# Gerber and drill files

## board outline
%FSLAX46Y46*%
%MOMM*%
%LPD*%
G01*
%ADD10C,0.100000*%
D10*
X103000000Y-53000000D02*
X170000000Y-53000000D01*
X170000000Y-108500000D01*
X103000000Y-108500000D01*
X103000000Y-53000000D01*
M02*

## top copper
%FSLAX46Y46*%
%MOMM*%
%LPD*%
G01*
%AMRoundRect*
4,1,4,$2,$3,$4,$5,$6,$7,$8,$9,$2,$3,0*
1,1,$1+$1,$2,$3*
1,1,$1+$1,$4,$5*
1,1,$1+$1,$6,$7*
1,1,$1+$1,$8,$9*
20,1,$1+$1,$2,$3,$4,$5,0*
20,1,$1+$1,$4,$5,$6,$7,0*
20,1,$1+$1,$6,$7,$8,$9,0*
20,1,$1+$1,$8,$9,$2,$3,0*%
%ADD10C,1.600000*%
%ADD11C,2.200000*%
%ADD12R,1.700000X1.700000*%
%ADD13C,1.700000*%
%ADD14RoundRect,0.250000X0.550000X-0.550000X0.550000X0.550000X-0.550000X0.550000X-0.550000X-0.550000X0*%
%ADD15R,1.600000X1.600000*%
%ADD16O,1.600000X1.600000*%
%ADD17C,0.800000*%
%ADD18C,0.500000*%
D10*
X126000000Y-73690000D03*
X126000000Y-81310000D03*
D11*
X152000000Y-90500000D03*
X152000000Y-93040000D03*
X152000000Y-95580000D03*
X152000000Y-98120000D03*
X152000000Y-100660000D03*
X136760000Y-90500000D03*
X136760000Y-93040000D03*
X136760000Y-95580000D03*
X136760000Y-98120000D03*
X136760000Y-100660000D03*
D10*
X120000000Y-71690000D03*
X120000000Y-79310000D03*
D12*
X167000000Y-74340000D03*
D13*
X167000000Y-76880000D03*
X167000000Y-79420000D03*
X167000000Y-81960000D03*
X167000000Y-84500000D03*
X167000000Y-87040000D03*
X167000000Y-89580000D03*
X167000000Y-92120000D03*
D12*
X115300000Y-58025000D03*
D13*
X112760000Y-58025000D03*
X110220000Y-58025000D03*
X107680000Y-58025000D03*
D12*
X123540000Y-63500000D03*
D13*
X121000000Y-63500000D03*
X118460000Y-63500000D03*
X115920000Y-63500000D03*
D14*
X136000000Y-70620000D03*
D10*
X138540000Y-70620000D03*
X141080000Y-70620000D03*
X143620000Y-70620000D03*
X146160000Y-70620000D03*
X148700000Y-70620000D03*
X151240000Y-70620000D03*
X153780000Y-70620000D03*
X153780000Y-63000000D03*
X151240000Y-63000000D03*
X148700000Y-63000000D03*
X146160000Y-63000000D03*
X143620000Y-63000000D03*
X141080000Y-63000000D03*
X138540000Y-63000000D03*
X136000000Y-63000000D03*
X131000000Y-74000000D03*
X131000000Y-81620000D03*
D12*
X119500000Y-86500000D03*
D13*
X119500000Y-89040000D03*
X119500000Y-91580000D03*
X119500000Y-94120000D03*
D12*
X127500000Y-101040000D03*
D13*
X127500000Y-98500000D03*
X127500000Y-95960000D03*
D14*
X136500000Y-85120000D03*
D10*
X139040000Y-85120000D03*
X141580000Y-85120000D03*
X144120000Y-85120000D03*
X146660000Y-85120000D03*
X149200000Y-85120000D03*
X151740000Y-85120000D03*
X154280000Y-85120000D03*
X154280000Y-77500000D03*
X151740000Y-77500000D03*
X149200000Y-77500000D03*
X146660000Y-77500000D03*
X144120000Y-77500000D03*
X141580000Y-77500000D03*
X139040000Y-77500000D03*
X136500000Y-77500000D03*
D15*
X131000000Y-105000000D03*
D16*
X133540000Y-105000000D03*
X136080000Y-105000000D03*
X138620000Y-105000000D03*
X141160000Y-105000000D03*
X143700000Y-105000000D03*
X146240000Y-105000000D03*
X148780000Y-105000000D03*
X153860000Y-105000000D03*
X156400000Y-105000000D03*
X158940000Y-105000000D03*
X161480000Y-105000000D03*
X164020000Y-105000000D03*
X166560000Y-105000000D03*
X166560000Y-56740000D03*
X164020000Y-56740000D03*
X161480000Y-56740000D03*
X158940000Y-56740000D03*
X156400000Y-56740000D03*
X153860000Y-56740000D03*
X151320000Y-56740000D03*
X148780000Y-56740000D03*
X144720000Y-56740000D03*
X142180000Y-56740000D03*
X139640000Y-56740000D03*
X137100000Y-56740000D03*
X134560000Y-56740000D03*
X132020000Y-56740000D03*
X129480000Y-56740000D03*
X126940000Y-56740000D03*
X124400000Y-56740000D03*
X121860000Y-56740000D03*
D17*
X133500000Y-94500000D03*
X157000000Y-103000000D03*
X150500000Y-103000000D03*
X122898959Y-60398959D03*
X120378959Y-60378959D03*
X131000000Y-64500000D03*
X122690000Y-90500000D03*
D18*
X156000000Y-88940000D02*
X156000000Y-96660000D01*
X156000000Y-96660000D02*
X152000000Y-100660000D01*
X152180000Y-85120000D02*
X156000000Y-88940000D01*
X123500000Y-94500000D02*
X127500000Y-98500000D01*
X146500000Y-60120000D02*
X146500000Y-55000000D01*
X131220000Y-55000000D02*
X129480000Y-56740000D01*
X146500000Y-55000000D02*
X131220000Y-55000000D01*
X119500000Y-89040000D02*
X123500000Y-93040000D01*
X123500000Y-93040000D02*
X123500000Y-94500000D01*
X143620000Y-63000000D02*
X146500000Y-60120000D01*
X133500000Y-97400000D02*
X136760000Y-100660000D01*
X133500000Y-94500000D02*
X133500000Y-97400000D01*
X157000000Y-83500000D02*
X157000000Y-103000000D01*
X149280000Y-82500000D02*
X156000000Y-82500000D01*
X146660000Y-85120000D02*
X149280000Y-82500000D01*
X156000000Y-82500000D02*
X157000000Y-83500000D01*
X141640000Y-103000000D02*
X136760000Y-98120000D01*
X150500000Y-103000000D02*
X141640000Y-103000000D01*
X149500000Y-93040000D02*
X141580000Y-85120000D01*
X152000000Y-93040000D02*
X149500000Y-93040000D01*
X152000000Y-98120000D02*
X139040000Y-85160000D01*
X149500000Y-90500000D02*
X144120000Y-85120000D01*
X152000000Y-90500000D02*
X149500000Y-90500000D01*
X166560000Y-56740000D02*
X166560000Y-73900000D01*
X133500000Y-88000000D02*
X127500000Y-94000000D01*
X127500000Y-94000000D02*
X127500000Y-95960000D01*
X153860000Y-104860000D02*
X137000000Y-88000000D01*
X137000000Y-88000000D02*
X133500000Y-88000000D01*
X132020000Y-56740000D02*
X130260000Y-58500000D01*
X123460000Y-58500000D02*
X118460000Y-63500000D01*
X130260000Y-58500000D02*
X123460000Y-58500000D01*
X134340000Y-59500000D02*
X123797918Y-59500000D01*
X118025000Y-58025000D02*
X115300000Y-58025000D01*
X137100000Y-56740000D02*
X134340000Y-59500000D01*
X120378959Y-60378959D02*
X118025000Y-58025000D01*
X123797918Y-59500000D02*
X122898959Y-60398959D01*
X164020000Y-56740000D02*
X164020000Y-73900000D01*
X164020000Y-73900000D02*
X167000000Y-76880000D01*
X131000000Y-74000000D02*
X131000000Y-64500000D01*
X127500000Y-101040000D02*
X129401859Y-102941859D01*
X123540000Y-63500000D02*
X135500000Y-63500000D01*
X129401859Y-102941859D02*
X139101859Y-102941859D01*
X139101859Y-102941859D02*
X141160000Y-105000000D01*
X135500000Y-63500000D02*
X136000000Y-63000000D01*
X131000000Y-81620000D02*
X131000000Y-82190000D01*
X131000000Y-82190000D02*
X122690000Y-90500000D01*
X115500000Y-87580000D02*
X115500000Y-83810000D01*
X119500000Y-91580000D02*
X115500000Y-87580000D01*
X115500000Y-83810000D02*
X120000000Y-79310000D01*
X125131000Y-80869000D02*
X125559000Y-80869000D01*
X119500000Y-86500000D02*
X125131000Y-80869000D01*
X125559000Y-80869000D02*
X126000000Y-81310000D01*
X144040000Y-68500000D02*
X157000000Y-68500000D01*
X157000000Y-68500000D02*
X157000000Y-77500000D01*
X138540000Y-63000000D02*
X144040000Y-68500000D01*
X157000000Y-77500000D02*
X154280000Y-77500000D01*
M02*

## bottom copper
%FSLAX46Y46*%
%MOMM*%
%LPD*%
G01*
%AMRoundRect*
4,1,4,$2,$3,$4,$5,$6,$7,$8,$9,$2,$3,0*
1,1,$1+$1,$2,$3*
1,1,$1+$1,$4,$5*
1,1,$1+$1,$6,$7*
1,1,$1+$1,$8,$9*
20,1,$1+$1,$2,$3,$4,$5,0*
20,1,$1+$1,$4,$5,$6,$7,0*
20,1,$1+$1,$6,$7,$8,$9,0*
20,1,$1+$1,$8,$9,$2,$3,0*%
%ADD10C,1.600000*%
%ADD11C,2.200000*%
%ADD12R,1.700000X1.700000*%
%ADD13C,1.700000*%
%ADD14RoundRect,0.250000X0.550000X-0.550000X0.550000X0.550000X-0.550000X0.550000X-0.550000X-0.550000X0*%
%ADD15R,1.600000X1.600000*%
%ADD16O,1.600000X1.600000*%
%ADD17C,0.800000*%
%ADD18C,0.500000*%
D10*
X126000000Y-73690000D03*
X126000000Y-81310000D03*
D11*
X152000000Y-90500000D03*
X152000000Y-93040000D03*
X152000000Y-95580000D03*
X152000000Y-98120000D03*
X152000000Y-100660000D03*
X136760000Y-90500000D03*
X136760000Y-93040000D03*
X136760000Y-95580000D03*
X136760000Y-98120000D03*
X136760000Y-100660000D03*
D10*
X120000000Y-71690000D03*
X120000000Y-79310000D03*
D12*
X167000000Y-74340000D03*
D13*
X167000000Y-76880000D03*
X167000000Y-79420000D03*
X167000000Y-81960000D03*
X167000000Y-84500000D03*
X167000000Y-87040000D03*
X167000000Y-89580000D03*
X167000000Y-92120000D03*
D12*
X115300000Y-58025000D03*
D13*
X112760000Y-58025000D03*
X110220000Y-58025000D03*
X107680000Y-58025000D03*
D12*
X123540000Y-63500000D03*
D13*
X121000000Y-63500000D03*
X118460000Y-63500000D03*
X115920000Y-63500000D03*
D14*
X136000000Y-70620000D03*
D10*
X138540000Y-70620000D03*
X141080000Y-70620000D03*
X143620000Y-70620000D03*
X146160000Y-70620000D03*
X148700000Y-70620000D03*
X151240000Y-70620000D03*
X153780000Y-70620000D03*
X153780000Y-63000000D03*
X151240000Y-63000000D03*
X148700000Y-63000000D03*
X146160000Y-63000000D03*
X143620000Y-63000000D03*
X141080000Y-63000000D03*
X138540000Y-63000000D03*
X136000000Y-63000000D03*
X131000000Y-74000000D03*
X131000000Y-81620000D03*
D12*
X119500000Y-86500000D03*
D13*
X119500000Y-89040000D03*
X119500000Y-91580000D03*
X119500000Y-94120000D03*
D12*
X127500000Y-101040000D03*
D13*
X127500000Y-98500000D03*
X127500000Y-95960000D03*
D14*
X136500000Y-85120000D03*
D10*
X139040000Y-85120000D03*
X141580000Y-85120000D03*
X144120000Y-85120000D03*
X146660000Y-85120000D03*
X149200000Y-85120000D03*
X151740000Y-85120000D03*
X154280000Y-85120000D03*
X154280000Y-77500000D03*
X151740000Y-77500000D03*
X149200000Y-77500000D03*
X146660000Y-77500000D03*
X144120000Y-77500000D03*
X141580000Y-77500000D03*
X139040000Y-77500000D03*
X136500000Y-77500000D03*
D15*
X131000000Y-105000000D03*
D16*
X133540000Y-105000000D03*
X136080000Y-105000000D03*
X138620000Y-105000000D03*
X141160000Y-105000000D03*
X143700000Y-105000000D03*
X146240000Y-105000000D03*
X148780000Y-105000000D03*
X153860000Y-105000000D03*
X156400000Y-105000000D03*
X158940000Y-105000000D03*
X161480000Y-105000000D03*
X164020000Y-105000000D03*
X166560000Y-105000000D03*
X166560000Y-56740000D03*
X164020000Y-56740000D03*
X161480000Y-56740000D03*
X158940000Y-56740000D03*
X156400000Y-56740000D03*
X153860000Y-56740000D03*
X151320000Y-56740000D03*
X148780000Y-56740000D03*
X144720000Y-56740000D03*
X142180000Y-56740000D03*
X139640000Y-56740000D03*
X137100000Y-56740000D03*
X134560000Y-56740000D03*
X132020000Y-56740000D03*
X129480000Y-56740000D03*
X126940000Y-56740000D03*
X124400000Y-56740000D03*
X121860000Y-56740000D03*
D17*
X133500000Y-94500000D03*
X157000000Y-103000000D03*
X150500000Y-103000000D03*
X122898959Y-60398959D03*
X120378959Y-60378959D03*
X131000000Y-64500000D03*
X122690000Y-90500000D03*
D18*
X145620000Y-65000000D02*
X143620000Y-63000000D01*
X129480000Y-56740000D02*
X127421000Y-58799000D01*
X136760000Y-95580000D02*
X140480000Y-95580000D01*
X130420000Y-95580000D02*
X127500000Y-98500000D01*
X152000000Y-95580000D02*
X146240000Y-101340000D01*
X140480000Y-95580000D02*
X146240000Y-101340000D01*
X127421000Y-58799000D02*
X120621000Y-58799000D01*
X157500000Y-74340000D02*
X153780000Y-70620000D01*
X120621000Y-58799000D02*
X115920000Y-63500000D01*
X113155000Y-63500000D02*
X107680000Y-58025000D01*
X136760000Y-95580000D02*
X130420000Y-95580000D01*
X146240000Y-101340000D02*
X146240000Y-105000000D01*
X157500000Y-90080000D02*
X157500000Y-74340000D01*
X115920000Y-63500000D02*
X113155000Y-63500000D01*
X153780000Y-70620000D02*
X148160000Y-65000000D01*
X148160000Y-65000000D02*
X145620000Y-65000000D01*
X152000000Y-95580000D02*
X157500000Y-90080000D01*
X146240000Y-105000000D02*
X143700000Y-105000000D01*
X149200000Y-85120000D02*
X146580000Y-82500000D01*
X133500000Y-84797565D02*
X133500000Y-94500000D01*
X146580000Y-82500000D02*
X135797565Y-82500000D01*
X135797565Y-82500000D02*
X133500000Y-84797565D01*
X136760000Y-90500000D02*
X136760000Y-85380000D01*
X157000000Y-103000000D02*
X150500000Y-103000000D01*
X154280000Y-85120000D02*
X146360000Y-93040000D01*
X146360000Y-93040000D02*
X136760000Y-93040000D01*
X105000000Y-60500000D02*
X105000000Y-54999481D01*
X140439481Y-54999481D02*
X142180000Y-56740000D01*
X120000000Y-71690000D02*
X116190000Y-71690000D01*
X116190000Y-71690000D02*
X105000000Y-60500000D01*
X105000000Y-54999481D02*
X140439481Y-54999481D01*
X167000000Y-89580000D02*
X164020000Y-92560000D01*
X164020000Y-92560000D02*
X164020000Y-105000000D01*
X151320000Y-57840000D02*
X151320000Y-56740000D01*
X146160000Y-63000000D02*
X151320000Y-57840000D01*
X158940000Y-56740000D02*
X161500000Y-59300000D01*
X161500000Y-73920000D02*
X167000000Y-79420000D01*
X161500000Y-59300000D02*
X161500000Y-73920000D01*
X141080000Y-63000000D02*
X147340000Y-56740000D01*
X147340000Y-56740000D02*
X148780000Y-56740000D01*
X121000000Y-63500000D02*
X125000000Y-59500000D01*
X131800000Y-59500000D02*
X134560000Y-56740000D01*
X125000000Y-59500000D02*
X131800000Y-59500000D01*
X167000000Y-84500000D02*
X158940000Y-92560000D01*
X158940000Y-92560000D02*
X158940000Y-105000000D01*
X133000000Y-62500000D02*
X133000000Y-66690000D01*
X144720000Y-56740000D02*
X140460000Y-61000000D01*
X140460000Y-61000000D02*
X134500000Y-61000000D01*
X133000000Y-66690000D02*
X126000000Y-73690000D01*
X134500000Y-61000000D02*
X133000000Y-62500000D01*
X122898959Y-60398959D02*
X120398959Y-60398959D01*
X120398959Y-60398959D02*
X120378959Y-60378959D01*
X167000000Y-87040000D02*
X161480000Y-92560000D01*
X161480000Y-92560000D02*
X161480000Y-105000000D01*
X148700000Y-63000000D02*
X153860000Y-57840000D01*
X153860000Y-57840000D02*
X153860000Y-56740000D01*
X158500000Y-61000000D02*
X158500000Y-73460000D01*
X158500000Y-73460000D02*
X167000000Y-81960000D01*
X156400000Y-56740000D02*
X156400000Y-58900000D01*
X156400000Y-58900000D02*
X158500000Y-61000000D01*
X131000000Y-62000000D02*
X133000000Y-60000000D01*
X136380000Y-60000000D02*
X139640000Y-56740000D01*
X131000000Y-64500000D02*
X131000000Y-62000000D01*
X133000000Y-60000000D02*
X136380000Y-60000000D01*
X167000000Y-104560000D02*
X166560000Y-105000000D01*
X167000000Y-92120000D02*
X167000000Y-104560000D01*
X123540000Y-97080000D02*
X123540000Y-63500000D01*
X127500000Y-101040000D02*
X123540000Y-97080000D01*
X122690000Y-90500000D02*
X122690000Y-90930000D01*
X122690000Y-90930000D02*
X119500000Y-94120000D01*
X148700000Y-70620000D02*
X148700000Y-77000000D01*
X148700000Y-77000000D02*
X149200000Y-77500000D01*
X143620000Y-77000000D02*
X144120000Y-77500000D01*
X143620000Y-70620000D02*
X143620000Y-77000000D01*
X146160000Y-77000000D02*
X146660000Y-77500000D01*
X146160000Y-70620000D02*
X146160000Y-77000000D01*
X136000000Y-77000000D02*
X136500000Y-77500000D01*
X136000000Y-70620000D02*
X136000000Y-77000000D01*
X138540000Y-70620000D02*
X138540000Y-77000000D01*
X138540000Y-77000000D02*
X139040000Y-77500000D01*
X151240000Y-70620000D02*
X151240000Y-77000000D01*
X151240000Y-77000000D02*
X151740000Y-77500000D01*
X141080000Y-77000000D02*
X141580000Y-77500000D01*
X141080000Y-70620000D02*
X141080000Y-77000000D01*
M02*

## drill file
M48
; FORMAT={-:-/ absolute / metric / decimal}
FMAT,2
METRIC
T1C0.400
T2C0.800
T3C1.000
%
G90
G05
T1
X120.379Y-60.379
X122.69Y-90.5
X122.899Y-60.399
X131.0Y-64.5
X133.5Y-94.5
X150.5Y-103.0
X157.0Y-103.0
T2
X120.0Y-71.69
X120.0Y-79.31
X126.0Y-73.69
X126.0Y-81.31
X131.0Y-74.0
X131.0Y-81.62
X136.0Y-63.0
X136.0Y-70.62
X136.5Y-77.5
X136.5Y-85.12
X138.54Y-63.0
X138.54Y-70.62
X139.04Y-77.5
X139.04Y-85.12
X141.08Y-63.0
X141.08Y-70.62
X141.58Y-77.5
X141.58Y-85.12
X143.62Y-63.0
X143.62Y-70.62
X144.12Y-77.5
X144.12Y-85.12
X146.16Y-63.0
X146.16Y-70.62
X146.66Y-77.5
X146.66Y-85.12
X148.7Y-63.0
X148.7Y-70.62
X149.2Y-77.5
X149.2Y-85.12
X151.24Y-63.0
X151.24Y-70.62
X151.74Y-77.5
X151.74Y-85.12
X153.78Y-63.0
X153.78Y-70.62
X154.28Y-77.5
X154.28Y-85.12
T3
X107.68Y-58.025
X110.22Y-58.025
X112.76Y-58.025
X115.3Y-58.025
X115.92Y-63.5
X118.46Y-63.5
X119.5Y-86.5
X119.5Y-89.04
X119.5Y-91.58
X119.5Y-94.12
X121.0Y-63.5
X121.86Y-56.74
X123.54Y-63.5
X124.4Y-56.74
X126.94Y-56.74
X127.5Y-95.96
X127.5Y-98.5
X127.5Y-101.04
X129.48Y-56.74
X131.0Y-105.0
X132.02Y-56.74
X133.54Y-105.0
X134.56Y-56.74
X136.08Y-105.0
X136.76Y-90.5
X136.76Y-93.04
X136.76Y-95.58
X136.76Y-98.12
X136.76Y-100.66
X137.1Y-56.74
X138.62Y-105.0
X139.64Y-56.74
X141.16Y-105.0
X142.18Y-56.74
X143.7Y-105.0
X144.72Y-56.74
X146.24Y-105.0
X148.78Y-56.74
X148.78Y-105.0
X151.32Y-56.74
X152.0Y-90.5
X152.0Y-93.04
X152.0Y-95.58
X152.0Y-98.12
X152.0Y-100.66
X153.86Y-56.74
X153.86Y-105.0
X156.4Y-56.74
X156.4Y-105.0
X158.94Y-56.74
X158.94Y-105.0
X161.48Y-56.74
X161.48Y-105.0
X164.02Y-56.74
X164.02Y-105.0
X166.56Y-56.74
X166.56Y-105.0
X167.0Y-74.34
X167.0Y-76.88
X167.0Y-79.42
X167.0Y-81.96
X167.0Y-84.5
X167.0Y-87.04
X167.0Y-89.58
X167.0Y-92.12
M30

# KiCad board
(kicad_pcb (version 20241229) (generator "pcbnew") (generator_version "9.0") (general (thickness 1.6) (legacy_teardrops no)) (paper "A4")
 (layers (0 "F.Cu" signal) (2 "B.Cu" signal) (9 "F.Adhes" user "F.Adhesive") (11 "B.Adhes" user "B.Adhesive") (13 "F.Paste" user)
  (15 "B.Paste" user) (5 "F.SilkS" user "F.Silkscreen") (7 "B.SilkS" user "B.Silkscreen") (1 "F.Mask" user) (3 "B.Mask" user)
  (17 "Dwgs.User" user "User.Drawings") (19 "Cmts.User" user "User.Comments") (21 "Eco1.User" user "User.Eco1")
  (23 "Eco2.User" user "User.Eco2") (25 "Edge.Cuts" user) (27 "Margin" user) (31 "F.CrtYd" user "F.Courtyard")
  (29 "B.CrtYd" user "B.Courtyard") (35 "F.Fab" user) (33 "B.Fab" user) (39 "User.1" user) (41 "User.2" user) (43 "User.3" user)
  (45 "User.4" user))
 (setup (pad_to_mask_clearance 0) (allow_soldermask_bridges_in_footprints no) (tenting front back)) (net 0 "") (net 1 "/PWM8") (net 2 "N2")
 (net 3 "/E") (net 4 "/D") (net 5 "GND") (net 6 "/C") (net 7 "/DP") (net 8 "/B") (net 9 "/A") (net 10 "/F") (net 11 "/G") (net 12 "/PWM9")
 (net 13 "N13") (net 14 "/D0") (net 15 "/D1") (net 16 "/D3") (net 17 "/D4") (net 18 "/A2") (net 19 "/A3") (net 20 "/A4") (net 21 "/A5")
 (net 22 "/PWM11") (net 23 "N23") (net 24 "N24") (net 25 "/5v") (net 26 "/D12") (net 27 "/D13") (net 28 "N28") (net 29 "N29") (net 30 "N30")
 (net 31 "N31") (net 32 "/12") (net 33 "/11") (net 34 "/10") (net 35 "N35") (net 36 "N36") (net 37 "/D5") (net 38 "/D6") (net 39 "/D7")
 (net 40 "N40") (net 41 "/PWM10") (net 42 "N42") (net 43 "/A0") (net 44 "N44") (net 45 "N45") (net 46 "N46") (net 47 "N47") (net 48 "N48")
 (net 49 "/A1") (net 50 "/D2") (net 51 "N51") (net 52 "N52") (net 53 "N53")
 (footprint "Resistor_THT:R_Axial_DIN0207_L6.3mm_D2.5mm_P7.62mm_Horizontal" (layer "F.Cu") (at 126 73.69 -90)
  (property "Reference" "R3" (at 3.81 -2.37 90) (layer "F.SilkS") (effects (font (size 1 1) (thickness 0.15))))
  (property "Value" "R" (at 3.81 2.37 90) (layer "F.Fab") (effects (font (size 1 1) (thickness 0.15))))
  (pad "1" thru_hole circle (at 0 0 270) (size 1.6 1.6) (drill 0.8) (layers "*.Cu" "*.Mask") (remove_unused_layers no) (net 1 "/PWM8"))
  (pad "2" thru_hole circle (at 7.62 0 270) (size 1.6 1.6) (drill 0.8) (layers "*.Cu" "*.Mask") (remove_unused_layers no) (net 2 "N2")))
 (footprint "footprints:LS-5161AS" (layer "F.Cu") (at 152 90.5 -90)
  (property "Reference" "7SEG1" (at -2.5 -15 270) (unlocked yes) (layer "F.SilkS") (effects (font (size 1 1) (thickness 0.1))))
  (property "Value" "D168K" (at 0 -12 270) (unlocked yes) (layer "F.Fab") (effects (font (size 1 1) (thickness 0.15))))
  (pad "1" thru_hole circle (at 0 0 270) (size 2.2 2.2) (drill 1) (layers "*.Cu" "*.Mask") (remove_unused_layers no) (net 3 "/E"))
  (pad "2" thru_hole circle (at 2.54 0 270) (size 2.2 2.2) (drill 1) (layers "*.Cu" "*.Mask") (remove_unused_layers no) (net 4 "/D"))
  (pad "3" thru_hole circle (at 5.08 0 270) (size 2.2 2.2) (drill 1) (layers "*.Cu" "*.Mask") (remove_unused_layers no) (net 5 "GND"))
  (pad "4" thru_hole circle (at 7.62 0 270) (size 2.2 2.2) (drill 1) (layers "*.Cu" "*.Mask") (remove_unused_layers no) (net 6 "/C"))
  (pad "5" thru_hole circle (at 10.16 0 270) (size 2.2 2.2) (drill 1) (layers "*.Cu" "*.Mask") (remove_unused_layers no) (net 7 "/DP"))
  (pad "6" thru_hole circle (at 0 15.24 270) (size 2.2 2.2) (drill 1) (layers "*.Cu" "*.Mask") (remove_unused_layers no) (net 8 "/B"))
  (pad "7" thru_hole circle (at 2.54 15.24 270) (size 2.2 2.2) (drill 1) (layers "*.Cu" "*.Mask") (remove_unused_layers no) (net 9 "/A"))
  (pad "8" thru_hole circle (at 5.08 15.24 270) (size 2.2 2.2) (drill 1) (layers "*.Cu" "*.Mask") (remove_unused_layers no) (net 5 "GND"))
  (pad "9" thru_hole circle (at 7.62 15.24 270) (size 2.2 2.2) (drill 1) (layers "*.Cu" "*.Mask") (remove_unused_layers no) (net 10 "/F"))
  (pad "10" thru_hole circle (at 10.16 15.24 270) (size 2.2 2.2) (drill 1) (layers "*.Cu" "*.Mask") (remove_unused_layers no) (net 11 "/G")))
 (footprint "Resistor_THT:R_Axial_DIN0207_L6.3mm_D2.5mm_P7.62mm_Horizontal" (layer "F.Cu") (at 120 71.69 -90)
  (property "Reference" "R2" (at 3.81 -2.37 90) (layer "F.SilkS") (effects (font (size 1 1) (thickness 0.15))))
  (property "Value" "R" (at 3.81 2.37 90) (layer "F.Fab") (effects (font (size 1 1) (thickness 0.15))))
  (pad "1" thru_hole circle (at 0 0 270) (size 1.6 1.6) (drill 0.8) (layers "*.Cu" "*.Mask") (remove_unused_layers no) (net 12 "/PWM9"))
  (pad "2" thru_hole circle (at 7.62 0 270) (size 1.6 1.6) (drill 0.8) (layers "*.Cu" "*.Mask") (remove_unused_layers no) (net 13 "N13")))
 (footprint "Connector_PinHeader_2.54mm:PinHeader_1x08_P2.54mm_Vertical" (layer "F.Cu") (at 167 74.34)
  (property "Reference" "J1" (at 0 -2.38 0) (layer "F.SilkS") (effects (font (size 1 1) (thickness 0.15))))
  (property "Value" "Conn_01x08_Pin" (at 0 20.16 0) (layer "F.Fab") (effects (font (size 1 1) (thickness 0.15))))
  (pad "1" thru_hole rect (at 0 0) (size 1.7 1.7) (drill 1) (layers "*.Cu" "*.Mask") (remove_unused_layers no) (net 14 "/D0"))
  (pad "2" thru_hole circle (at 0 2.54) (size 1.7 1.7) (drill 1) (layers "*.Cu" "*.Mask") (remove_unused_layers no) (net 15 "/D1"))
  (pad "3" thru_hole circle (at 0 5.08) (size 1.7 1.7) (drill 1) (layers "*.Cu" "*.Mask") (remove_unused_layers no) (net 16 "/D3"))
  (pad "4" thru_hole circle (at 0 7.62) (size 1.7 1.7) (drill 1) (layers "*.Cu" "*.Mask") (remove_unused_layers no) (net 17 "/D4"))
  (pad "5" thru_hole circle (at 0 10.16) (size 1.7 1.7) (drill 1) (layers "*.Cu" "*.Mask") (remove_unused_layers no) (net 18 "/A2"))
  (pad "6" thru_hole circle (at 0 12.7) (size 1.7 1.7) (drill 1) (layers "*.Cu" "*.Mask") (remove_unused_layers no) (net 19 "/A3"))
  (pad "7" thru_hole circle (at 0 15.24) (size 1.7 1.7) (drill 1) (layers "*.Cu" "*.Mask") (remove_unused_layers no) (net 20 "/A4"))
  (pad "8" thru_hole circle (at 0 17.78) (size 1.7 1.7) (drill 1) (layers "*.Cu" "*.Mask") (remove_unused_layers no) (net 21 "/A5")))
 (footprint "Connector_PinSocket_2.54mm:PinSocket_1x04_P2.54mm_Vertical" (layer "F.Cu") (at 115.3 58.025 -90)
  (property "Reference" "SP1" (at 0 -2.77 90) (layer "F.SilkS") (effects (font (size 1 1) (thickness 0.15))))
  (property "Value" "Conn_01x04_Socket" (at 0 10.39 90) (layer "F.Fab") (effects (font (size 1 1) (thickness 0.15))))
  (pad "1" thru_hole rect (at 0 0 270) (size 1.7 1.7) (drill 1) (layers "*.Cu" "*.Mask") (remove_unused_layers no) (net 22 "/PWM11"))
  (pad "2" thru_hole circle (at 0 2.54 270) (size 1.7 1.7) (drill 1) (layers "*.Cu" "*.Mask") (remove_unused_layers no) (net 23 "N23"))
  (pad "3" thru_hole circle (at 0 5.08 270) (size 1.7 1.7) (drill 1) (layers "*.Cu" "*.Mask") (remove_unused_layers no) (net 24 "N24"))
  (pad "4" thru_hole circle (at 0 7.62 270) (size 1.7 1.7) (drill 1) (layers "*.Cu" "*.Mask") (remove_unused_layers no) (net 5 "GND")))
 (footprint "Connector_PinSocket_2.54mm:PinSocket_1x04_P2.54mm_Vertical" (layer "F.Cu") (at 123.54 63.5 -90)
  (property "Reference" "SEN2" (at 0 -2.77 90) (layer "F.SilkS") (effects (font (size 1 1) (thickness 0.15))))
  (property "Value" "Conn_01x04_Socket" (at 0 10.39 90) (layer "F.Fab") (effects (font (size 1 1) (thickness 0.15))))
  (pad "1" thru_hole rect (at 0 0 270) (size 1.7 1.7) (drill 1) (layers "*.Cu" "*.Mask") (remove_unused_layers no) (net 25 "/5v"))
  (pad "2" thru_hole circle (at 0 2.54 270) (size 1.7 1.7) (drill 1) (layers "*.Cu" "*.Mask") (remove_unused_layers no) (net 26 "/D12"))
  (pad "3" thru_hole circle (at 0 5.08 270) (size 1.7 1.7) (drill 1) (layers "*.Cu" "*.Mask") (remove_unused_layers no) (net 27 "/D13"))
  (pad "4" thru_hole circle (at 0 7.62 270) (size 1.7 1.7) (drill 1) (layers "*.Cu" "*.Mask") (remove_unused_layers no) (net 5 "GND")))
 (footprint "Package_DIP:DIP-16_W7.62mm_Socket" (layer "F.Cu") (at 136 70.62 90)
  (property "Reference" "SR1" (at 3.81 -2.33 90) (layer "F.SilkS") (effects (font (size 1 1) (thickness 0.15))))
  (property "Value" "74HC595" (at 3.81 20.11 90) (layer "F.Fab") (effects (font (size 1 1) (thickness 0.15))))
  (pad "1" thru_hole roundrect (at 0 0 90) (size 1.6 1.6) (drill 0.8) (layers "*.Cu" "*.Mask") (remove_unused_layers no)
   (roundrect_rratio 0.15625) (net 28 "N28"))
  (pad "2" thru_hole circle (at 0 2.54 90) (size 1.6 1.6) (drill 0.8) (layers "*.Cu" "*.Mask") (remove_unused_layers no) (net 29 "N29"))
  (pad "3" thru_hole circle (at 0 5.08 90) (size 1.6 1.6) (drill 0.8) (layers "*.Cu" "*.Mask") (remove_unused_layers no) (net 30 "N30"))
  (pad "4" thru_hole circle (at 0 7.62 90) (size 1.6 1.6) (drill 0.8) (layers "*.Cu" "*.Mask") (remove_unused_layers no) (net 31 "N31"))
  (pad "5" thru_hole circle (at 0 10.16 90) (size 1.6 1.6) (drill 0.8) (layers "*.Cu" "*.Mask") (remove_unused_layers no) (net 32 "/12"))
  (pad "6" thru_hole circle (at 0 12.7 90) (size 1.6 1.6) (drill 0.8) (layers "*.Cu" "*.Mask") (remove_unused_layers no) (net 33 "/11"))
  (pad "7" thru_hole circle (at 0 15.24 90) (size 1.6 1.6) (drill 0.8) (layers "*.Cu" "*.Mask") (remove_unused_layers no) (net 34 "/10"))
  (pad "8" thru_hole circle (at 0 17.78 90) (size 1.6 1.6) (drill 0.8) (layers "*.Cu" "*.Mask") (remove_unused_layers no) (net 5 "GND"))
  (pad "9" thru_hole circle (at 7.62 17.78 90) (size 1.6 1.6) (drill 0.8) (layers "*.Cu" "*.Mask") (remove_unused_layers no) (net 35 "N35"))
  (pad "10" thru_hole circle (at 7.62 15.24 90) (size 1.6 1.6) (drill 0.8) (layers "*.Cu" "*.Mask") (remove_unused_layers no) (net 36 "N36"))
  (pad "11" thru_hole circle (at 7.62 12.7 90) (size 1.6 1.6) (drill 0.8) (layers "*.Cu" "*.Mask") (remove_unused_layers no) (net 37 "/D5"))
  (pad "12" thru_hole circle (at 7.62 10.16 90) (size 1.6 1.6) (drill 0.8) (layers "*.Cu" "*.Mask") (remove_unused_layers no) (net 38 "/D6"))
  (pad "13" thru_hole circle (at 7.62 7.62 90) (size 1.6 1.6) (drill 0.8) (layers "*.Cu" "*.Mask") (remove_unused_layers no) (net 5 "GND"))
  (pad "14" thru_hole circle (at 7.62 5.08 90) (size 1.6 1.6) (drill 0.8) (layers "*.Cu" "*.Mask") (remove_unused_layers no) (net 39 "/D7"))
  (pad "15" thru_hole circle (at 7.62 2.54 90) (size 1.6 1.6) (drill 0.8) (layers "*.Cu" "*.Mask") (remove_unused_layers no) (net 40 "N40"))
  (pad "16" thru_hole circle (at 7.62 0 90) (size 1.6 1.6) (drill 0.8) (layers "*.Cu" "*.Mask") (remove_unused_layers no) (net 25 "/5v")))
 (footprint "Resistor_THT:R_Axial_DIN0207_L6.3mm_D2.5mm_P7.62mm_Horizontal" (layer "F.Cu") (at 131 74 -90)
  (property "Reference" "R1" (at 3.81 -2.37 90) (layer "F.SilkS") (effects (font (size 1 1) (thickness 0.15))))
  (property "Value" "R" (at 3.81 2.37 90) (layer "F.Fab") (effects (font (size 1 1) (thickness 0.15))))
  (pad "1" thru_hole circle (at 0 0 270) (size 1.6 1.6) (drill 0.8) (layers "*.Cu" "*.Mask") (remove_unused_layers no) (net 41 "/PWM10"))
  (pad "2" thru_hole circle (at 7.62 0 270) (size 1.6 1.6) (drill 0.8) (layers "*.Cu" "*.Mask") (remove_unused_layers no) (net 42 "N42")))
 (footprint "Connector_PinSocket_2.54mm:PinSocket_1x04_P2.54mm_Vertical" (layer "F.Cu") (at 119.5 86.5)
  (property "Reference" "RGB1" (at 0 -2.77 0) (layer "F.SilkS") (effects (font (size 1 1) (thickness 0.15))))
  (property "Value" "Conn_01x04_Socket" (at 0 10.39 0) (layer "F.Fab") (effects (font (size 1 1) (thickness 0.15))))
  (pad "1" thru_hole rect (at 0 0) (size 1.7 1.7) (drill 1) (layers "*.Cu" "*.Mask") (remove_unused_layers no) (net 2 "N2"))
  (pad "2" thru_hole circle (at 0 2.54) (size 1.7 1.7) (drill 1) (layers "*.Cu" "*.Mask") (remove_unused_layers no) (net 5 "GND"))
  (pad "3" thru_hole circle (at 0 5.08) (size 1.7 1.7) (drill 1) (layers "*.Cu" "*.Mask") (remove_unused_layers no) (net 13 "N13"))
  (pad "4" thru_hole circle (at 0 7.62) (size 1.7 1.7) (drill 1) (layers "*.Cu" "*.Mask") (remove_unused_layers no) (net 42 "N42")))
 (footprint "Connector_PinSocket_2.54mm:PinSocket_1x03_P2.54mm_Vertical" (layer "F.Cu") (at 127.5 101.04 180)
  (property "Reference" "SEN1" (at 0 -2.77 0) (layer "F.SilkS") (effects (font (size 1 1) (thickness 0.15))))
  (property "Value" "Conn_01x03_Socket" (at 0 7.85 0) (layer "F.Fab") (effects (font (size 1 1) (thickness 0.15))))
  (pad "1" thru_hole rect (at 0 0 180) (size 1.7 1.7) (drill 1) (layers "*.Cu" "*.Mask") (remove_unused_layers no) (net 25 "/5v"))
  (pad "2" thru_hole circle (at 0 2.54 180) (size 1.7 1.7) (drill 1) (layers "*.Cu" "*.Mask") (remove_unused_layers no) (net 5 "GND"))
  (pad "3" thru_hole circle (at 0 5.08 180) (size 1.7 1.7) (drill 1) (layers "*.Cu" "*.Mask") (remove_unused_layers no) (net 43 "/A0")))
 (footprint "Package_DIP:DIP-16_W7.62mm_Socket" (layer "F.Cu") (at 136.5 85.12 90)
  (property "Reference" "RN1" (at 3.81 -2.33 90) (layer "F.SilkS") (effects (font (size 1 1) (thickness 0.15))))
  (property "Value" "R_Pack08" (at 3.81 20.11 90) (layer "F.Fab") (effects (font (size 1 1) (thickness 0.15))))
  (pad "1" thru_hole roundrect (at 0 0 90) (size 1.6 1.6) (drill 0.8) (layers "*.Cu" "*.Mask") (remove_unused_layers no)
   (roundrect_rratio 0.15625) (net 8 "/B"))
  (pad "2" thru_hole circle (at 0 2.54 90) (size 1.6 1.6) (drill 0.8) (layers "*.Cu" "*.Mask") (remove_unused_layers no) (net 6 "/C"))
  (pad "3" thru_hole circle (at 0 5.08 90) (size 1.6 1.6) (drill 0.8) (layers "*.Cu" "*.Mask") (remove_unused_layers no) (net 4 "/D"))
  (pad "4" thru_hole circle (at 0 7.62 90) (size 1.6 1.6) (drill 0.8) (layers "*.Cu" "*.Mask") (remove_unused_layers no) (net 3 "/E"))
  (pad "5" thru_hole circle (at 0 10.16 90) (size 1.6 1.6) (drill 0.8) (layers "*.Cu" "*.Mask") (remove_unused_layers no) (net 10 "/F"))
  (pad "6" thru_hole circle (at 0 12.7 90) (size 1.6 1.6) (drill 0.8) (layers "*.Cu" "*.Mask") (remove_unused_layers no) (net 11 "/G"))
  (pad "7" thru_hole circle (at 0 15.24 90) (size 1.6 1.6) (drill 0.8) (layers "*.Cu" "*.Mask") (remove_unused_layers no) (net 7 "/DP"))
  (pad "8" thru_hole circle (at 0 17.78 90) (size 1.6 1.6) (drill 0.8) (layers "*.Cu" "*.Mask") (remove_unused_layers no) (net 9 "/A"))
  (pad "9" thru_hole circle (at 7.62 17.78 90) (size 1.6 1.6) (drill 0.8) (layers "*.Cu" "*.Mask") (remove_unused_layers no) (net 40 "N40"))
  (pad "10" thru_hole circle (at 7.62 15.24 90) (size 1.6 1.6) (drill 0.8) (layers "*.Cu" "*.Mask") (remove_unused_layers no) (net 34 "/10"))
  (pad "11" thru_hole circle (at 7.62 12.7 90) (size 1.6 1.6) (drill 0.8) (layers "*.Cu" "*.Mask") (remove_unused_layers no) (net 33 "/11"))
  (pad "12" thru_hole circle (at 7.62 10.16 90) (size 1.6 1.6) (drill 0.8) (layers "*.Cu" "*.Mask") (remove_unused_layers no) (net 32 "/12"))
  (pad "13" thru_hole circle (at 7.62 7.62 90) (size 1.6 1.6) (drill 0.8) (layers "*.Cu" "*.Mask") (remove_unused_layers no) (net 31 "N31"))
  (pad "14" thru_hole circle (at 7.62 5.08 90) (size 1.6 1.6) (drill 0.8) (layers "*.Cu" "*.Mask") (remove_unused_layers no) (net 30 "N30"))
  (pad "15" thru_hole circle (at 7.62 2.54 90) (size 1.6 1.6) (drill 0.8) (layers "*.Cu" "*.Mask") (remove_unused_layers no) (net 29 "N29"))
  (pad "16" thru_hole circle (at 7.62 0 90) (size 1.6 1.6) (drill 0.8) (layers "*.Cu" "*.Mask") (remove_unused_layers no) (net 28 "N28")))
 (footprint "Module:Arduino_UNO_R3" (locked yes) (layer "B.Cu") (at 131 105)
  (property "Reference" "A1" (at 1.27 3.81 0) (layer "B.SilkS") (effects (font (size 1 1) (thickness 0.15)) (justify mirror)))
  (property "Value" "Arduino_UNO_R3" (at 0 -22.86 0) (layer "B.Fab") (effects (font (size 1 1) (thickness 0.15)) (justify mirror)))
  (pad "1" thru_hole rect (at 0 0 270) (size 1.6 1.6) (drill 1) (layers "*.Cu" "*.Mask") (remove_unused_layers no) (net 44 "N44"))
  (pad "2" thru_hole oval (at 2.54 0 270) (size 1.6 1.6) (drill 1) (layers "*.Cu" "*.Mask") (remove_unused_layers no) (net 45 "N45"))
  (pad "3" thru_hole oval (at 5.08 0 270) (size 1.6 1.6) (drill 1) (layers "*.Cu" "*.Mask") (remove_unused_layers no) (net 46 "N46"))
  (pad "4" thru_hole oval (at 7.62 0 270) (size 1.6 1.6) (drill 1) (layers "*.Cu" "*.Mask") (remove_unused_layers no) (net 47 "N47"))
  (pad "5" thru_hole oval (at 10.16 0 270) (size 1.6 1.6) (drill 1) (layers "*.Cu" "*.Mask") (remove_unused_layers no) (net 25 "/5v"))
  (pad "6" thru_hole oval (at 12.7 0 270) (size 1.6 1.6) (drill 1) (layers "*.Cu" "*.Mask") (remove_unused_layers no) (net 5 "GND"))
  (pad "7" thru_hole oval (at 15.24 0 270) (size 1.6 1.6) (drill 1) (layers "*.Cu" "*.Mask") (remove_unused_layers no) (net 5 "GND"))
  (pad "8" thru_hole oval (at 17.78 0 270) (size 1.6 1.6) (drill 1) (layers "*.Cu" "*.Mask") (remove_unused_layers no) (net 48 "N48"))
  (pad "9" thru_hole oval (at 22.86 0 270) (size 1.6 1.6) (drill 1) (layers "*.Cu" "*.Mask") (remove_unused_layers no) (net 43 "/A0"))
  (pad "10" thru_hole oval (at 25.4 0 270) (size 1.6 1.6) (drill 1) (layers "*.Cu" "*.Mask") (remove_unused_layers no) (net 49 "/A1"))
  (pad "11" thru_hole oval (at 27.94 0 270) (size 1.6 1.6) (drill 1) (layers "*.Cu" "*.Mask") (remove_unused_layers no) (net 18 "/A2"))
  (pad "12" thru_hole oval (at 30.48 0 270) (size 1.6 1.6) (drill 1) (layers "*.Cu" "*.Mask") (remove_unused_layers no) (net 19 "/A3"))
  (pad "13" thru_hole oval (at 33.02 0 270) (size 1.6 1.6) (drill 1) (layers "*.Cu" "*.Mask") (remove_unused_layers no) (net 20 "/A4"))
  (pad "14" thru_hole oval (at 35.56 0 270) (size 1.6 1.6) (drill 1) (layers "*.Cu" "*.Mask") (remove_unused_layers no) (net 21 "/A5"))
  (pad "15" thru_hole oval (at 35.56 -48.26 270) (size 1.6 1.6) (drill 1) (layers "*.Cu" "*.Mask") (remove_unused_layers no) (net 14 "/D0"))
  (pad "16" thru_hole oval (at 33.02 -48.26 270) (size 1.6 1.6) (drill 1) (layers "*.Cu" "*.Mask") (remove_unused_layers no) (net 15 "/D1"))
  (pad "17" thru_hole oval (at 30.48 -48.26 270) (size 1.6 1.6) (drill 1) (layers "*.Cu" "*.Mask") (remove_unused_layers no) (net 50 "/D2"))
  (pad "18" thru_hole oval (at 27.94 -48.26 270) (size 1.6 1.6) (drill 1) (layers "*.Cu" "*.Mask") (remove_unused_layers no) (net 16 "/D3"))
  (pad "19" thru_hole oval (at 25.4 -48.26 270) (size 1.6 1.6) (drill 1) (layers "*.Cu" "*.Mask") (remove_unused_layers no) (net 17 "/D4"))
  (pad "20" thru_hole oval (at 22.86 -48.26 270) (size 1.6 1.6) (drill 1) (layers "*.Cu" "*.Mask") (remove_unused_layers no) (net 37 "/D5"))
  (pad "21" thru_hole oval (at 20.32 -48.26 270) (size 1.6 1.6) (drill 1) (layers "*.Cu" "*.Mask") (remove_unused_layers no) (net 38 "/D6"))
  (pad "22" thru_hole oval (at 17.78 -48.26 270) (size 1.6 1.6) (drill 1) (layers "*.Cu" "*.Mask") (remove_unused_layers no) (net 39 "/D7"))
  (pad "23" thru_hole oval (at 13.72 -48.26 270) (size 1.6 1.6) (drill 1) (layers "*.Cu" "*.Mask") (remove_unused_layers no) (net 1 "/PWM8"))
  (pad "24" thru_hole oval (at 11.18 -48.26 270) (size 1.6 1.6) (drill 1) (layers "*.Cu" "*.Mask") (remove_unused_layers no)
   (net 12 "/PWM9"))
  (pad "25" thru_hole oval (at 8.64 -48.26 270) (size 1.6 1.6) (drill 1) (layers "*.Cu" "*.Mask") (remove_unused_layers no)
   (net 41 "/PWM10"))
  (pad "26" thru_hole oval (at 6.1 -48.26 270) (size 1.6 1.6) (drill 1) (layers "*.Cu" "*.Mask") (remove_unused_layers no) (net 22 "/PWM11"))
  (pad "27" thru_hole oval (at 3.56 -48.26 270) (size 1.6 1.6) (drill 1) (layers "*.Cu" "*.Mask") (remove_unused_layers no) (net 26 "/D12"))
  (pad "28" thru_hole oval (at 1.02 -48.26 270) (size 1.6 1.6) (drill 1) (layers "*.Cu" "*.Mask") (remove_unused_layers no) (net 27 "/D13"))
  (pad "29" thru_hole oval (at -1.52 -48.26 270) (size 1.6 1.6) (drill 1) (layers "*.Cu" "*.Mask") (remove_unused_layers no) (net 5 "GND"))
  (pad "30" thru_hole oval (at -4.06 -48.26 270) (size 1.6 1.6) (drill 1) (layers "*.Cu" "*.Mask") (remove_unused_layers no) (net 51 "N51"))
  (pad "31" thru_hole oval (at -6.6 -48.26 270) (size 1.6 1.6) (drill 1) (layers "*.Cu" "*.Mask") (remove_unused_layers no) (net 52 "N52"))
  (pad "32" thru_hole oval (at -9.14 -48.26 270) (size 1.6 1.6) (drill 1) (layers "*.Cu" "*.Mask") (remove_unused_layers no) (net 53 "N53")))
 (gr_rect (start 103 53) (end 170 108.5) (stroke (width 0.1) (type default)) (fill no) (layer "Edge.Cuts"))
 (segment (start 156 88.94) (end 156 96.66) (width 0.5) (layer "F.Cu") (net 7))
 (segment (start 156 96.66) (end 152 100.66) (width 0.5) (layer "F.Cu") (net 7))
 (segment (start 152.18 85.12) (end 156 88.94) (width 0.5) (layer "F.Cu") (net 7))
 (segment (start 123.5 94.5) (end 127.5 98.5) (width 0.5) (layer "F.Cu") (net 5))
 (segment (start 146.5 60.12) (end 146.5 55) (width 0.5) (layer "F.Cu") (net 5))
 (segment (start 131.22 55) (end 129.48 56.74) (width 0.5) (layer "F.Cu") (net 5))
 (segment (start 146.5 55) (end 131.22 55) (width 0.5) (layer "F.Cu") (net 5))
 (segment (start 119.5 89.04) (end 123.5 93.04) (width 0.5) (layer "F.Cu") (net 5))
 (segment (start 123.5 93.04) (end 123.5 94.5) (width 0.5) (layer "F.Cu") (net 5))
 (segment (start 143.62 63) (end 146.5 60.12) (width 0.5) (layer "F.Cu") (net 5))
 (segment (start 145.62 65) (end 143.62 63) (width 0.5) (layer "B.Cu") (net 5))
 (segment (start 129.48 56.74) (end 127.421 58.799) (width 0.5) (layer "B.Cu") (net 5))
 (segment (start 136.76 95.58) (end 140.48 95.58) (width 0.5) (layer "B.Cu") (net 5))
 (segment (start 130.42 95.58) (end 127.5 98.5) (width 0.5) (layer "B.Cu") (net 5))
 (segment (start 152 95.58) (end 146.24 101.34) (width 0.5) (layer "B.Cu") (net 5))
 (segment (start 140.48 95.58) (end 146.24 101.34) (width 0.5) (layer "B.Cu") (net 5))
 (segment (start 127.421 58.799) (end 120.621 58.799) (width 0.5) (layer "B.Cu") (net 5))
 (segment (start 157.5 74.34) (end 153.78 70.62) (width 0.5) (layer "B.Cu") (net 5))
 (segment (start 120.621 58.799) (end 115.92 63.5) (width 0.5) (layer "B.Cu") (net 5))
 (segment (start 113.155 63.5) (end 107.68 58.025) (width 0.5) (layer "B.Cu") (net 5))
 (segment (start 136.76 95.58) (end 130.42 95.58) (width 0.5) (layer "B.Cu") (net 5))
 (segment (start 146.24 101.34) (end 146.24 105) (width 0.5) (layer "B.Cu") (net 5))
 (segment (start 157.5 90.08) (end 157.5 74.34) (width 0.5) (layer "B.Cu") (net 5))
 (segment (start 115.92 63.5) (end 113.155 63.5) (width 0.5) (layer "B.Cu") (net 5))
 (segment (start 153.78 70.62) (end 148.16 65) (width 0.5) (layer "B.Cu") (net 5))
 (segment (start 148.16 65) (end 145.62 65) (width 0.5) (layer "B.Cu") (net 5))
 (segment (start 152 95.58) (end 157.5 90.08) (width 0.5) (layer "B.Cu") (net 5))
 (segment (start 146.24 105) (end 143.7 105) (width 0.5) (layer "B.Cu") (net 5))
 (segment (start 133.5 97.4) (end 136.76 100.66) (width 0.5) (layer "F.Cu") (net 11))
 (segment (start 133.5 94.5) (end 133.5 97.4) (width 0.5) (layer "F.Cu") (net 11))
 (via (at 133.5 94.5) (size 0.8) (drill 0.4) (layers "F.Cu" "B.Cu") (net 11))
 (segment (start 149.2 85.12) (end 146.58 82.5) (width 0.5) (layer "B.Cu") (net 11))
 (segment (start 133.5 84.797565) (end 133.5 94.5) (width 0.5) (layer "B.Cu") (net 11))
 (segment (start 146.58 82.5) (end 135.797565 82.5) (width 0.5) (layer "B.Cu") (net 11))
 (segment (start 135.797565 82.5) (end 133.5 84.797565) (width 0.5) (layer "B.Cu") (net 11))
 (segment (start 136.76 90.5) (end 136.76 85.38) (width 0.5) (layer "B.Cu") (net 8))
 (segment (start 157 83.5) (end 157 103) (width 0.5) (layer "F.Cu") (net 10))
 (segment (start 149.28 82.5) (end 156 82.5) (width 0.5) (layer "F.Cu") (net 10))
 (segment (start 146.66 85.12) (end 149.28 82.5) (width 0.5) (layer "F.Cu") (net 10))
 (segment (start 156 82.5) (end 157 83.5) (width 0.5) (layer "F.Cu") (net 10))
 (segment (start 141.64 103) (end 136.76 98.12) (width 0.5) (layer "F.Cu") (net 10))
 (segment (start 150.5 103) (end 141.64 103) (width 0.5) (layer "F.Cu") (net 10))
 (via (at 157 103) (size 0.8) (drill 0.4) (layers "F.Cu" "B.Cu") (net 10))
 (via (at 150.5 103) (size 0.8) (drill 0.4) (layers "F.Cu" "B.Cu") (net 10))
 (segment (start 157 103) (end 150.5 103) (width 0.5) (layer "B.Cu") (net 10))
 (segment (start 149.5 93.04) (end 141.58 85.12) (width 0.5) (layer "F.Cu") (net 4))
 (segment (start 152 93.04) (end 149.5 93.04) (width 0.5) (layer "F.Cu") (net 4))
 (segment (start 152 98.12) (end 139.04 85.16) (width 0.5) (layer "F.Cu") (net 6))
 (segment (start 154.28 85.12) (end 146.36 93.04) (width 0.5) (layer "B.Cu") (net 9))
 (segment (start 146.36 93.04) (end 136.76 93.04) (width 0.5) (layer "B.Cu") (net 9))
 (segment (start 149.5 90.5) (end 144.12 85.12) (width 0.5) (layer "F.Cu") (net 3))
 (segment (start 152 90.5) (end 149.5 90.5) (width 0.5) (layer "F.Cu") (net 3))
 (segment (start 105 60.5) (end 105 54.999481) (width 0.5) (layer "B.Cu") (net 12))
 (segment (start 140.439481 54.999481) (end 142.18 56.74) (width 0.5) (layer "B.Cu") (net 12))
 (segment (start 120 71.69) (end 116.19 71.69) (width 0.5) (layer "B.Cu") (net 12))
 (segment (start 116.19 71.69) (end 105 60.5) (width 0.5) (layer "B.Cu") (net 12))
 (segment (start 105 54.999481) (end 140.439481 54.999481) (width 0.5) (layer "B.Cu") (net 12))
 (segment (start 167 89.58) (end 164.02 92.56) (width 0.5) (layer "B.Cu") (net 20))
 (segment (start 164.02 92.56) (end 164.02 105) (width 0.5) (layer "B.Cu") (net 20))
 (segment (start 151.32 57.84) (end 151.32 56.74) (width 0.5) (layer "B.Cu") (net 38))
 (segment (start 146.16 63) (end 151.32 57.84) (width 0.5) (layer "B.Cu") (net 38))
 (segment (start 166.56 56.74) (end 166.56 73.9) (width 0.5) (layer "F.Cu") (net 14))
 (segment (start 133.5 88) (end 127.5 94) (width 0.5) (layer "F.Cu") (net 43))
 (segment (start 127.5 94) (end 127.5 95.96) (width 0.5) (layer "F.Cu") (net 43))
 (segment (start 153.86 104.86) (end 137 88) (width 0.5) (layer "F.Cu") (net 43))
 (segment (start 137 88) (end 133.5 88) (width 0.5) (layer "F.Cu") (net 43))
 (segment (start 158.94 56.74) (end 161.5 59.3) (width 0.5) (layer "B.Cu") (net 16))
 (segment (start 161.5 73.92) (end 167 79.42) (width 0.5) (layer "B.Cu") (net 16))
 (segment (start 161.5 59.3) (end 161.5 73.92) (width 0.5) (layer "B.Cu") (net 16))
 (segment (start 141.08 63) (end 147.34 56.74) (width 0.5) (layer "B.Cu") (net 39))
 (segment (start 147.34 56.74) (end 148.78 56.74) (width 0.5) (layer "B.Cu") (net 39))
 (segment (start 121 63.5) (end 125 59.5) (width 0.5) (layer "B.Cu") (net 26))
 (segment (start 131.8 59.5) (end 134.56 56.74) (width 0.5) (layer "B.Cu") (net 26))
 (segment (start 125 59.5) (end 131.8 59.5) (width 0.5) (layer "B.Cu") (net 26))
 (segment (start 167 84.5) (end 158.94 92.56) (width 0.5) (layer "B.Cu") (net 18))
 (segment (start 158.94 92.56) (end 158.94 105) (width 0.5) (layer "B.Cu") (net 18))
 (segment (start 133 62.5) (end 133 66.69) (width 0.5) (layer "B.Cu") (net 1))
 (segment (start 144.72 56.74) (end 140.46 61) (width 0.5) (layer "B.Cu") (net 1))
 (segment (start 140.46 61) (end 134.5 61) (width 0.5) (layer "B.Cu") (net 1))
 (segment (start 133 66.69) (end 126 73.69) (width 0.5) (layer "B.Cu") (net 1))
 (segment (start 134.5 61) (end 133 62.5) (width 0.5) (layer "B.Cu") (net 1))
 (segment (start 132.02 56.74) (end 130.26 58.5) (width 0.5) (layer "F.Cu") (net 27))
 (segment (start 123.46 58.5) (end 118.46 63.5) (width 0.5) (layer "F.Cu") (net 27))
 (segment (start 130.26 58.5) (end 123.46 58.5) (width 0.5) (layer "F.Cu") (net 27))
 (segment (start 134.34 59.5) (end 123.797918 59.5) (width 0.5) (layer "F.Cu") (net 22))
 (segment (start 118.025 58.025) (end 115.3 58.025) (width 0.5) (layer "F.Cu") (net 22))
 (segment (start 137.1 56.74) (end 134.34 59.5) (width 0.5) (layer "F.Cu") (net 22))
 (segment (start 120.378959 60.378959) (end 118.025 58.025) (width 0.5) (layer "F.Cu") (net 22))
 (segment (start 123.797918 59.5) (end 122.898959 60.398959) (width 0.5) (layer "F.Cu") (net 22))
 (via (at 122.898959 60.398959) (size 0.8) (drill 0.4) (layers "F.Cu" "B.Cu") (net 22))
 (via (at 120.378959 60.378959) (size 0.8) (drill 0.4) (layers "F.Cu" "B.Cu") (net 22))
 (segment (start 122.898959 60.398959) (end 120.398959 60.398959) (width 0.5) (layer "B.Cu") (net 22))
 (segment (start 120.398959 60.398959) (end 120.378959 60.378959) (width 0.5) (layer "B.Cu") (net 22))
 (segment (start 167 87.04) (end 161.48 92.56) (width 0.5) (layer "B.Cu") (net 19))
 (segment (start 161.48 92.56) (end 161.48 105) (width 0.5) (layer "B.Cu") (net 19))
 (segment (start 148.7 63) (end 153.86 57.84) (width 0.5) (layer "B.Cu") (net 37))
 (segment (start 153.86 57.84) (end 153.86 56.74) (width 0.5) (layer "B.Cu") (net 37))
 (segment (start 164.02 56.74) (end 164.02 73.9) (width 0.5) (layer "F.Cu") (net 15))
 (segment (start 164.02 73.9) (end 167 76.88) (width 0.5) (layer "F.Cu") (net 15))
 (segment (start 158.5 61) (end 158.5 73.46) (width 0.5) (layer "B.Cu") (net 17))
 (segment (start 158.5 73.46) (end 167 81.96) (width 0.5) (layer "B.Cu") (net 17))
 (segment (start 156.4 56.74) (end 156.4 58.9) (width 0.5) (layer "B.Cu") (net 17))
 (segment (start 156.4 58.9) (end 158.5 61) (width 0.5) (layer "B.Cu") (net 17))
 (segment (start 131 74) (end 131 64.5) (width 0.5) (layer "F.Cu") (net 41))
 (via (at 131 64.5) (size 0.8) (drill 0.4) (layers "F.Cu" "B.Cu") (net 41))
 (segment (start 131 62) (end 133 60) (width 0.5) (layer "B.Cu") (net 41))
 (segment (start 136.38 60) (end 139.64 56.74) (width 0.5) (layer "B.Cu") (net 41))
 (segment (start 131 64.5) (end 131 62) (width 0.5) (layer "B.Cu") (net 41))
 (segment (start 133 60) (end 136.38 60) (width 0.5) (layer "B.Cu") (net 41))
 (segment (start 167 104.56) (end 166.56 105) (width 0.5) (layer "B.Cu") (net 21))
 (segment (start 167 92.12) (end 167 104.56) (width 0.5) (layer "B.Cu") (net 21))
 (segment (start 127.5 101.04) (end 129.401859 102.941859) (width 0.5) (layer "F.Cu") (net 25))
 (segment (start 123.54 63.5) (end 135.5 63.5) (width 0.5) (layer "F.Cu") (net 25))
 (segment (start 129.401859 102.941859) (end 139.101859 102.941859) (width 0.5) (layer "F.Cu") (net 25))
 (segment (start 139.101859 102.941859) (end 141.16 105) (width 0.5) (layer "F.Cu") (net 25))
 (segment (start 135.5 63.5) (end 136 63) (width 0.5) (layer "F.Cu") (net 25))
 (segment (start 123.54 97.08) (end 123.54 63.5) (width 0.5) (layer "B.Cu") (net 25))
 (segment (start 127.5 101.04) (end 123.54 97.08) (width 0.5) (layer "B.Cu") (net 25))
 (segment (start 131 81.62) (end 131 82.19) (width 0.5) (layer "F.Cu") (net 42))
 (segment (start 131 82.19) (end 122.69 90.5) (width 0.5) (layer "F.Cu") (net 42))
 (via (at 122.69 90.5) (size 0.8) (drill 0.4) (layers "F.Cu" "B.Cu") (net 42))
 (segment (start 122.69 90.5) (end 122.69 90.93) (width 0.5) (layer "B.Cu") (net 42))
 (segment (start 122.69 90.93) (end 119.5 94.12) (width 0.5) (layer "B.Cu") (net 42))
 (segment (start 115.5 87.58) (end 115.5 83.81) (width 0.5) (layer "F.Cu") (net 13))
 (segment (start 119.5 91.58) (end 115.5 87.58) (width 0.5) (layer "F.Cu") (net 13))
 (segment (start 115.5 83.81) (end 120 79.31) (width 0.5) (layer "F.Cu") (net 13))
 (segment (start 125.131 80.869) (end 125.559 80.869) (width 0.5) (layer "F.Cu") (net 2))
 (segment (start 119.5 86.5) (end 125.131 80.869) (width 0.5) (layer "F.Cu") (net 2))
 (segment (start 125.559 80.869) (end 126 81.31) (width 0.5) (layer "F.Cu") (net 2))
 (segment (start 144.04 68.5) (end 157 68.5) (width 0.5) (layer "F.Cu") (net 40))
 (segment (start 157 68.5) (end 157 77.5) (width 0.5) (layer "F.Cu") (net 40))
 (segment (start 138.54 63) (end 144.04 68.5) (width 0.5) (layer "F.Cu") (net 40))
 (segment (start 157 77.5) (end 154.28 77.5) (width 0.5) (layer "F.Cu") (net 40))
 (segment (start 148.7 70.62) (end 148.7 77) (width 0.5) (layer "B.Cu") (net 33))
 (segment (start 148.7 77) (end 149.2 77.5) (width 0.5) (layer "B.Cu") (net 33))
 (segment (start 143.62 77) (end 144.12 77.5) (width 0.5) (layer "B.Cu") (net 31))
 (segment (start 143.62 70.62) (end 143.62 77) (width 0.5) (layer "B.Cu") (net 31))
 (segment (start 146.16 77) (end 146.66 77.5) (width 0.5) (layer "B.Cu") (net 32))
 (segment (start 146.16 70.62) (end 146.16 77) (width 0.5) (layer "B.Cu") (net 32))
 (segment (start 136 77) (end 136.5 77.5) (width 0.5) (layer "B.Cu") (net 28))
 (segment (start 136 70.62) (end 136 77) (width 0.5) (layer "B.Cu") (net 28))
 (segment (start 138.54 70.62) (end 138.54 77) (width 0.5) (layer "B.Cu") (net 29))
 (segment (start 138.54 77) (end 139.04 77.5) (width 0.5) (layer "B.Cu") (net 29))
 (segment (start 151.24 70.62) (end 151.24 77) (width 0.5) (layer "B.Cu") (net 34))
 (segment (start 151.24 77) (end 151.74 77.5) (width 0.5) (layer "B.Cu") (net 34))
 (segment (start 141.08 77) (end 141.58 77.5) (width 0.5) (layer "B.Cu") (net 30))
 (segment (start 141.08 70.62) (end 141.08 77) (width 0.5) (layer "B.Cu") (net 30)))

